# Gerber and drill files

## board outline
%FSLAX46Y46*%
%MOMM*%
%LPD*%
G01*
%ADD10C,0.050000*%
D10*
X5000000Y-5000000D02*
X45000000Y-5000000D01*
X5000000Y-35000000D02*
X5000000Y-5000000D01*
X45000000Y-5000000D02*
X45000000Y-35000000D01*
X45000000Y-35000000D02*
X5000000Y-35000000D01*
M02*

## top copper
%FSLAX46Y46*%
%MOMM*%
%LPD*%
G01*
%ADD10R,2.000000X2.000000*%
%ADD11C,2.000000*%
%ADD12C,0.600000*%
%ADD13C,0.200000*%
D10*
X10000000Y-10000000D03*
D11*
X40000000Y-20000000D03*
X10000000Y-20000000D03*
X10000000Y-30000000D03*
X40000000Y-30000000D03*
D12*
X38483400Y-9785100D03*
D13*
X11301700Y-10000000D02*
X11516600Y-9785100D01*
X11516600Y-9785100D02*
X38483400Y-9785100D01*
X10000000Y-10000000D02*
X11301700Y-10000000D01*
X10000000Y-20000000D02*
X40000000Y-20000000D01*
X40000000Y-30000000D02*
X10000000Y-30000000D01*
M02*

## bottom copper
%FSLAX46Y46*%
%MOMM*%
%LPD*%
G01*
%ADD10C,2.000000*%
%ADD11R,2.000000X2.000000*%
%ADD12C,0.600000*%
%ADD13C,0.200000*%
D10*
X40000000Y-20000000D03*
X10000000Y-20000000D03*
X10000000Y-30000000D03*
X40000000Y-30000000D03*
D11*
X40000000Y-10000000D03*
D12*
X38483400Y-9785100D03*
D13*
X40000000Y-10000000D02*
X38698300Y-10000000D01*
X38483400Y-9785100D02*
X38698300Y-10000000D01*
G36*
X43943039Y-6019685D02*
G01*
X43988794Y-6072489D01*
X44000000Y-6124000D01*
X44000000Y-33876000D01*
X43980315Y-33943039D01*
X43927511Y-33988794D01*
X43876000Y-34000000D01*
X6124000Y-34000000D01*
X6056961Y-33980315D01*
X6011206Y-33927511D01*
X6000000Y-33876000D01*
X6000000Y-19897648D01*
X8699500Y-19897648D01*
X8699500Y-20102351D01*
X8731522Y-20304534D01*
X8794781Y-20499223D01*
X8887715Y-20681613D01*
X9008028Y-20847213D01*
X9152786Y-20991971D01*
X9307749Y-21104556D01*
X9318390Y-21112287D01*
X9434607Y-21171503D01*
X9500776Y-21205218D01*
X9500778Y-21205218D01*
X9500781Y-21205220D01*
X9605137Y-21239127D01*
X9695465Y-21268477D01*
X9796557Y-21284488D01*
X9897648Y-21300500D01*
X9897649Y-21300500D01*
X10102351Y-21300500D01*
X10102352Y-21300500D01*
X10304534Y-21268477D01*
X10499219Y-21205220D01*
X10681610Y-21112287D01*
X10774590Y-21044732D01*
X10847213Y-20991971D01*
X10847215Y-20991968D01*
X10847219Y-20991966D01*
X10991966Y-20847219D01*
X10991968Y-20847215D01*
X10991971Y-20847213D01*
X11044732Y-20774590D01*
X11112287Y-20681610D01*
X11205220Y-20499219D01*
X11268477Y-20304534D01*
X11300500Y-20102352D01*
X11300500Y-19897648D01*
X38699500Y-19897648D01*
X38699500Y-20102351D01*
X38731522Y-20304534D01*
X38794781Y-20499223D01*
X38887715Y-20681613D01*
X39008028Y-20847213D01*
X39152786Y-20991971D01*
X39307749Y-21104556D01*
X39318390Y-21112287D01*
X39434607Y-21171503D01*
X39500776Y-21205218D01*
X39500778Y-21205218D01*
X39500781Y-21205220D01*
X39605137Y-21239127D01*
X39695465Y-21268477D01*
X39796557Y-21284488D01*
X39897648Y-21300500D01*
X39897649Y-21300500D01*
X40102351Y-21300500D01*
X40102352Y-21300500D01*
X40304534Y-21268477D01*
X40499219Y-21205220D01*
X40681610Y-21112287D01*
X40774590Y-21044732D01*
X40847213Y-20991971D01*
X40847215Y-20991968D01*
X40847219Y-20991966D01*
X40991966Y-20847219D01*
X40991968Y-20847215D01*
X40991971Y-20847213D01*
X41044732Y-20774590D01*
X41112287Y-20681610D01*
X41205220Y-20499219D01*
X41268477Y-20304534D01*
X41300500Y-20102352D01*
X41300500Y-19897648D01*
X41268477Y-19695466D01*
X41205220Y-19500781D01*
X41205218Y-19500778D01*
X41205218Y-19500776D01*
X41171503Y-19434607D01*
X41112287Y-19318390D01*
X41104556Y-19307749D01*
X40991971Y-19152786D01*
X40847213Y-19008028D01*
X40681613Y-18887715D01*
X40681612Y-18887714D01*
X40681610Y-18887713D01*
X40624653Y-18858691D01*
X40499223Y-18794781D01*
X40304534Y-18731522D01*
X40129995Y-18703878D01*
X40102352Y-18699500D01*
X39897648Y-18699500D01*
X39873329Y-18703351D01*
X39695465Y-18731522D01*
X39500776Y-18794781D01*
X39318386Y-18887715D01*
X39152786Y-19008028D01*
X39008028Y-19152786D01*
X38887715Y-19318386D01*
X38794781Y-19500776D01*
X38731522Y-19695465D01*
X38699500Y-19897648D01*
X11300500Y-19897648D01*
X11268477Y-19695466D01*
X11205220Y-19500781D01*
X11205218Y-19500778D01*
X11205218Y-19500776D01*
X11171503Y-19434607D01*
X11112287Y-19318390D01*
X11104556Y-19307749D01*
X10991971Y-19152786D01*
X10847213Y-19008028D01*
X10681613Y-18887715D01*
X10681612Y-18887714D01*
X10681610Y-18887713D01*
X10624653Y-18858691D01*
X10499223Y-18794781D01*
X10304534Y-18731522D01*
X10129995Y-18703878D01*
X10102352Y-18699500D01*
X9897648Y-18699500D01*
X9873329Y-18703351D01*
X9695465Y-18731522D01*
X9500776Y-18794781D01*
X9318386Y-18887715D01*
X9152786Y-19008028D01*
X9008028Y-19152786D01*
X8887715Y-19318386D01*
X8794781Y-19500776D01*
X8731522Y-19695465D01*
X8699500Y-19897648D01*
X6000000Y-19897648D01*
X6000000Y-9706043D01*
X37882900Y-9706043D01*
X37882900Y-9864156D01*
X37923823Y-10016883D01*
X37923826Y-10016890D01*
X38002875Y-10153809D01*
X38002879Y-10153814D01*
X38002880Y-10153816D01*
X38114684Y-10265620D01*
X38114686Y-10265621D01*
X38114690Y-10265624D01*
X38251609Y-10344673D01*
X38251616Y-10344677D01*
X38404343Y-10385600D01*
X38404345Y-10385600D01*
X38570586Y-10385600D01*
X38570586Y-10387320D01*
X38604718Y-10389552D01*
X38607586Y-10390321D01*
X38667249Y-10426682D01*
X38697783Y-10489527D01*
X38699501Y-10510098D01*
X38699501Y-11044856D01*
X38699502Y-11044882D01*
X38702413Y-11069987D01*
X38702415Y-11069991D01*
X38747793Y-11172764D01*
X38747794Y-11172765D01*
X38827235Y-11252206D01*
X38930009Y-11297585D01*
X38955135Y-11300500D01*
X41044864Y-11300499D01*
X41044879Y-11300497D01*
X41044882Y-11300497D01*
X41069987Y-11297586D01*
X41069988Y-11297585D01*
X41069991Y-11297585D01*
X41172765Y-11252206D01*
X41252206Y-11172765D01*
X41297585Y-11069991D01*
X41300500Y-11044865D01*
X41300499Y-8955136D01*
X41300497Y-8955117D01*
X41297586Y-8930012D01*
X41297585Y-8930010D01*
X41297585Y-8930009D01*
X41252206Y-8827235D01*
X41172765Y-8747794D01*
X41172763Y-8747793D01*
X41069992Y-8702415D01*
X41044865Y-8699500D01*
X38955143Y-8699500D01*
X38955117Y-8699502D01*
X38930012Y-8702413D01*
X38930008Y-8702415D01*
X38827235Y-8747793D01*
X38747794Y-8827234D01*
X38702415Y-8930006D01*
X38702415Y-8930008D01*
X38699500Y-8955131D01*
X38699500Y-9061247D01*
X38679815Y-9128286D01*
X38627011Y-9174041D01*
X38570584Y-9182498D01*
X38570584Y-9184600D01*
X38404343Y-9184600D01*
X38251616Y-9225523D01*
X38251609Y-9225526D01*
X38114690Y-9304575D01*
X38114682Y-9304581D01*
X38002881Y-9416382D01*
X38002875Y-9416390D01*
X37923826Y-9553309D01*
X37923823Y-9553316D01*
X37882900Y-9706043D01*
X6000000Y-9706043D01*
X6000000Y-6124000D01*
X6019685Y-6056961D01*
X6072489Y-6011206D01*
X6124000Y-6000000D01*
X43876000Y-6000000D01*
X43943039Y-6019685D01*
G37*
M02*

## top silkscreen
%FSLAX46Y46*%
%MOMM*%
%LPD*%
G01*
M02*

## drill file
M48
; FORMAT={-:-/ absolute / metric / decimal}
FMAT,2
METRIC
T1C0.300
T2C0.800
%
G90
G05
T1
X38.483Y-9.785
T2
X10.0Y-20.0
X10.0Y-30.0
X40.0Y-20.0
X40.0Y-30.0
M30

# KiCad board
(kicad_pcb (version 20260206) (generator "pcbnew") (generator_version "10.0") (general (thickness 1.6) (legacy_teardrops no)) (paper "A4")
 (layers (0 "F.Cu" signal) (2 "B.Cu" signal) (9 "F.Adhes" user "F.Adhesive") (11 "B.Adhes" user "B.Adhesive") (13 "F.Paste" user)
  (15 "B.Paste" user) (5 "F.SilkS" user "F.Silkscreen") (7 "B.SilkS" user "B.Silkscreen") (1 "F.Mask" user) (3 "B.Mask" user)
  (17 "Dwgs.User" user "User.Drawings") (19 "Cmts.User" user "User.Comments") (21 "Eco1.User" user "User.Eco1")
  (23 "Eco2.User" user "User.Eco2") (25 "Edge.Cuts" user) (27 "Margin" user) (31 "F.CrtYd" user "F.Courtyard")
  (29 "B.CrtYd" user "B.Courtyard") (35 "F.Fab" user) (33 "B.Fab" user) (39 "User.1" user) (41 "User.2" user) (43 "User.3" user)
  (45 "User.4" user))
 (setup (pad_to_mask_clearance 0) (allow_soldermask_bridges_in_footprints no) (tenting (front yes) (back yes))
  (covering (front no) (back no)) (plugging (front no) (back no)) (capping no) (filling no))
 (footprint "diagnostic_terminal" (layer "F.Cu") (at 10 10)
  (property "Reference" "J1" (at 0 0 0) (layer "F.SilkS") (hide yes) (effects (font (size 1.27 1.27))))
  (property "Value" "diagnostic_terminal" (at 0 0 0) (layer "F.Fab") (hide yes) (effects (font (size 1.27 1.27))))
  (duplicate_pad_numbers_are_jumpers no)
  (pad "1" smd rect (at 0 0) (size 2 2) (layers "F.Cu") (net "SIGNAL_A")))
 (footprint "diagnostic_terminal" (layer "F.Cu") (at 40 20)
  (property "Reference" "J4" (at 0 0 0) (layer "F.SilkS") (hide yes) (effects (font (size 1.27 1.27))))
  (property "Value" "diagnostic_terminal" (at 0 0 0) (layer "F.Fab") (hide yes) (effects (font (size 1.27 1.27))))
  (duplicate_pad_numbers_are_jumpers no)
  (pad "1" thru_hole circle (at 0 0) (size 2 2) (drill 0.8) (layers "*.Cu") (remove_unused_layers no) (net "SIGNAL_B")))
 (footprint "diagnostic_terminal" (layer "F.Cu") (at 10 20)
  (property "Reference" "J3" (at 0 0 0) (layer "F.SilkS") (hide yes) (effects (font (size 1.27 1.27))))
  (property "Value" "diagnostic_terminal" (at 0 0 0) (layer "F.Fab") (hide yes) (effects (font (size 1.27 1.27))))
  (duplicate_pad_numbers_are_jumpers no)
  (pad "1" thru_hole circle (at 0 0) (size 2 2) (drill 0.8) (layers "*.Cu") (remove_unused_layers no) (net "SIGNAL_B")))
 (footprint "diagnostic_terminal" (layer "F.Cu") (at 10 30)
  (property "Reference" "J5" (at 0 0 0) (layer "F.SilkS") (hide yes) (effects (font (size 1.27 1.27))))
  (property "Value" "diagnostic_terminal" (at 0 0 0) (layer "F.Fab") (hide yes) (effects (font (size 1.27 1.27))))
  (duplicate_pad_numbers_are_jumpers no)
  (pad "1" thru_hole circle (at 0 0) (size 2 2) (drill 0.8) (layers "*.Cu") (remove_unused_layers no) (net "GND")))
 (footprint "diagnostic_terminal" (layer "F.Cu") (at 40 30)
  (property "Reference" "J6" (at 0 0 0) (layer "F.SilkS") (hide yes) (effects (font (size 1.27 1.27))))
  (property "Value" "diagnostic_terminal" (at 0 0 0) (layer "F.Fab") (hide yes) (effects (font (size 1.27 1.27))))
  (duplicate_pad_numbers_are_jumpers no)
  (pad "1" thru_hole circle (at 0 0) (size 2 2) (drill 0.8) (layers "*.Cu") (remove_unused_layers no) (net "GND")))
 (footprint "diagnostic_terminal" (layer "B.Cu") (at 40 10)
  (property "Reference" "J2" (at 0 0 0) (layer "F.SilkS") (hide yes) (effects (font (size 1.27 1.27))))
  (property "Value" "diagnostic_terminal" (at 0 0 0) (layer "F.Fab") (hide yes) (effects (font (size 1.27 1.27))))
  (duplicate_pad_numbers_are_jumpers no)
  (pad "1" smd rect (at 0 0) (size 2 2) (layers "B.Cu") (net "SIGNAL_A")))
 (gr_line (start 5 5) (end 45 5) (stroke (width 0.05) (type default)) (layer "Edge.Cuts"))
 (gr_line (start 5 35) (end 5 5) (stroke (width 0.05) (type default)) (layer "Edge.Cuts"))
 (gr_line (start 45 5) (end 45 35) (stroke (width 0.05) (type default)) (layer "Edge.Cuts"))
 (gr_line (start 45 35) (end 5 35) (stroke (width 0.05) (type default)) (layer "Edge.Cuts"))
 (segment (start 11.3017 10) (end 11.5166 9.7851) (width 0.2) (layer "F.Cu") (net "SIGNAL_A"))
 (segment (start 11.5166 9.7851) (end 38.4834 9.7851) (width 0.2) (layer "F.Cu") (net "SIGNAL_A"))
 (segment (start 10 10) (end 11.3017 10) (width 0.2) (layer "F.Cu") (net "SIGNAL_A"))
 (via (at 38.4834 9.7851) (size 0.6) (drill 0.3) (layers "F.Cu" "B.Cu") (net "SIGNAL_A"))
 (segment (start 40 10) (end 38.6983 10) (width 0.2) (layer "B.Cu") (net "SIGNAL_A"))
 (segment (start 38.4834 9.7851) (end 38.6983 10) (width 0.2) (layer "B.Cu") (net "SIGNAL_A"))
 (segment (start 10 20) (end 40 20) (width 0.2) (layer "F.Cu") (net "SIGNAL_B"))
 (segment (start 40 30) (end 10 30) (width 0.2) (layer "F.Cu") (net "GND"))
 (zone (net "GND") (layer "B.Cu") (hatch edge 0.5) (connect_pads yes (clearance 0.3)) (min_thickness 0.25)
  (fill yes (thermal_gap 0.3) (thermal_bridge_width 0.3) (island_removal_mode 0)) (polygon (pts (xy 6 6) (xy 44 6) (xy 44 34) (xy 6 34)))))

